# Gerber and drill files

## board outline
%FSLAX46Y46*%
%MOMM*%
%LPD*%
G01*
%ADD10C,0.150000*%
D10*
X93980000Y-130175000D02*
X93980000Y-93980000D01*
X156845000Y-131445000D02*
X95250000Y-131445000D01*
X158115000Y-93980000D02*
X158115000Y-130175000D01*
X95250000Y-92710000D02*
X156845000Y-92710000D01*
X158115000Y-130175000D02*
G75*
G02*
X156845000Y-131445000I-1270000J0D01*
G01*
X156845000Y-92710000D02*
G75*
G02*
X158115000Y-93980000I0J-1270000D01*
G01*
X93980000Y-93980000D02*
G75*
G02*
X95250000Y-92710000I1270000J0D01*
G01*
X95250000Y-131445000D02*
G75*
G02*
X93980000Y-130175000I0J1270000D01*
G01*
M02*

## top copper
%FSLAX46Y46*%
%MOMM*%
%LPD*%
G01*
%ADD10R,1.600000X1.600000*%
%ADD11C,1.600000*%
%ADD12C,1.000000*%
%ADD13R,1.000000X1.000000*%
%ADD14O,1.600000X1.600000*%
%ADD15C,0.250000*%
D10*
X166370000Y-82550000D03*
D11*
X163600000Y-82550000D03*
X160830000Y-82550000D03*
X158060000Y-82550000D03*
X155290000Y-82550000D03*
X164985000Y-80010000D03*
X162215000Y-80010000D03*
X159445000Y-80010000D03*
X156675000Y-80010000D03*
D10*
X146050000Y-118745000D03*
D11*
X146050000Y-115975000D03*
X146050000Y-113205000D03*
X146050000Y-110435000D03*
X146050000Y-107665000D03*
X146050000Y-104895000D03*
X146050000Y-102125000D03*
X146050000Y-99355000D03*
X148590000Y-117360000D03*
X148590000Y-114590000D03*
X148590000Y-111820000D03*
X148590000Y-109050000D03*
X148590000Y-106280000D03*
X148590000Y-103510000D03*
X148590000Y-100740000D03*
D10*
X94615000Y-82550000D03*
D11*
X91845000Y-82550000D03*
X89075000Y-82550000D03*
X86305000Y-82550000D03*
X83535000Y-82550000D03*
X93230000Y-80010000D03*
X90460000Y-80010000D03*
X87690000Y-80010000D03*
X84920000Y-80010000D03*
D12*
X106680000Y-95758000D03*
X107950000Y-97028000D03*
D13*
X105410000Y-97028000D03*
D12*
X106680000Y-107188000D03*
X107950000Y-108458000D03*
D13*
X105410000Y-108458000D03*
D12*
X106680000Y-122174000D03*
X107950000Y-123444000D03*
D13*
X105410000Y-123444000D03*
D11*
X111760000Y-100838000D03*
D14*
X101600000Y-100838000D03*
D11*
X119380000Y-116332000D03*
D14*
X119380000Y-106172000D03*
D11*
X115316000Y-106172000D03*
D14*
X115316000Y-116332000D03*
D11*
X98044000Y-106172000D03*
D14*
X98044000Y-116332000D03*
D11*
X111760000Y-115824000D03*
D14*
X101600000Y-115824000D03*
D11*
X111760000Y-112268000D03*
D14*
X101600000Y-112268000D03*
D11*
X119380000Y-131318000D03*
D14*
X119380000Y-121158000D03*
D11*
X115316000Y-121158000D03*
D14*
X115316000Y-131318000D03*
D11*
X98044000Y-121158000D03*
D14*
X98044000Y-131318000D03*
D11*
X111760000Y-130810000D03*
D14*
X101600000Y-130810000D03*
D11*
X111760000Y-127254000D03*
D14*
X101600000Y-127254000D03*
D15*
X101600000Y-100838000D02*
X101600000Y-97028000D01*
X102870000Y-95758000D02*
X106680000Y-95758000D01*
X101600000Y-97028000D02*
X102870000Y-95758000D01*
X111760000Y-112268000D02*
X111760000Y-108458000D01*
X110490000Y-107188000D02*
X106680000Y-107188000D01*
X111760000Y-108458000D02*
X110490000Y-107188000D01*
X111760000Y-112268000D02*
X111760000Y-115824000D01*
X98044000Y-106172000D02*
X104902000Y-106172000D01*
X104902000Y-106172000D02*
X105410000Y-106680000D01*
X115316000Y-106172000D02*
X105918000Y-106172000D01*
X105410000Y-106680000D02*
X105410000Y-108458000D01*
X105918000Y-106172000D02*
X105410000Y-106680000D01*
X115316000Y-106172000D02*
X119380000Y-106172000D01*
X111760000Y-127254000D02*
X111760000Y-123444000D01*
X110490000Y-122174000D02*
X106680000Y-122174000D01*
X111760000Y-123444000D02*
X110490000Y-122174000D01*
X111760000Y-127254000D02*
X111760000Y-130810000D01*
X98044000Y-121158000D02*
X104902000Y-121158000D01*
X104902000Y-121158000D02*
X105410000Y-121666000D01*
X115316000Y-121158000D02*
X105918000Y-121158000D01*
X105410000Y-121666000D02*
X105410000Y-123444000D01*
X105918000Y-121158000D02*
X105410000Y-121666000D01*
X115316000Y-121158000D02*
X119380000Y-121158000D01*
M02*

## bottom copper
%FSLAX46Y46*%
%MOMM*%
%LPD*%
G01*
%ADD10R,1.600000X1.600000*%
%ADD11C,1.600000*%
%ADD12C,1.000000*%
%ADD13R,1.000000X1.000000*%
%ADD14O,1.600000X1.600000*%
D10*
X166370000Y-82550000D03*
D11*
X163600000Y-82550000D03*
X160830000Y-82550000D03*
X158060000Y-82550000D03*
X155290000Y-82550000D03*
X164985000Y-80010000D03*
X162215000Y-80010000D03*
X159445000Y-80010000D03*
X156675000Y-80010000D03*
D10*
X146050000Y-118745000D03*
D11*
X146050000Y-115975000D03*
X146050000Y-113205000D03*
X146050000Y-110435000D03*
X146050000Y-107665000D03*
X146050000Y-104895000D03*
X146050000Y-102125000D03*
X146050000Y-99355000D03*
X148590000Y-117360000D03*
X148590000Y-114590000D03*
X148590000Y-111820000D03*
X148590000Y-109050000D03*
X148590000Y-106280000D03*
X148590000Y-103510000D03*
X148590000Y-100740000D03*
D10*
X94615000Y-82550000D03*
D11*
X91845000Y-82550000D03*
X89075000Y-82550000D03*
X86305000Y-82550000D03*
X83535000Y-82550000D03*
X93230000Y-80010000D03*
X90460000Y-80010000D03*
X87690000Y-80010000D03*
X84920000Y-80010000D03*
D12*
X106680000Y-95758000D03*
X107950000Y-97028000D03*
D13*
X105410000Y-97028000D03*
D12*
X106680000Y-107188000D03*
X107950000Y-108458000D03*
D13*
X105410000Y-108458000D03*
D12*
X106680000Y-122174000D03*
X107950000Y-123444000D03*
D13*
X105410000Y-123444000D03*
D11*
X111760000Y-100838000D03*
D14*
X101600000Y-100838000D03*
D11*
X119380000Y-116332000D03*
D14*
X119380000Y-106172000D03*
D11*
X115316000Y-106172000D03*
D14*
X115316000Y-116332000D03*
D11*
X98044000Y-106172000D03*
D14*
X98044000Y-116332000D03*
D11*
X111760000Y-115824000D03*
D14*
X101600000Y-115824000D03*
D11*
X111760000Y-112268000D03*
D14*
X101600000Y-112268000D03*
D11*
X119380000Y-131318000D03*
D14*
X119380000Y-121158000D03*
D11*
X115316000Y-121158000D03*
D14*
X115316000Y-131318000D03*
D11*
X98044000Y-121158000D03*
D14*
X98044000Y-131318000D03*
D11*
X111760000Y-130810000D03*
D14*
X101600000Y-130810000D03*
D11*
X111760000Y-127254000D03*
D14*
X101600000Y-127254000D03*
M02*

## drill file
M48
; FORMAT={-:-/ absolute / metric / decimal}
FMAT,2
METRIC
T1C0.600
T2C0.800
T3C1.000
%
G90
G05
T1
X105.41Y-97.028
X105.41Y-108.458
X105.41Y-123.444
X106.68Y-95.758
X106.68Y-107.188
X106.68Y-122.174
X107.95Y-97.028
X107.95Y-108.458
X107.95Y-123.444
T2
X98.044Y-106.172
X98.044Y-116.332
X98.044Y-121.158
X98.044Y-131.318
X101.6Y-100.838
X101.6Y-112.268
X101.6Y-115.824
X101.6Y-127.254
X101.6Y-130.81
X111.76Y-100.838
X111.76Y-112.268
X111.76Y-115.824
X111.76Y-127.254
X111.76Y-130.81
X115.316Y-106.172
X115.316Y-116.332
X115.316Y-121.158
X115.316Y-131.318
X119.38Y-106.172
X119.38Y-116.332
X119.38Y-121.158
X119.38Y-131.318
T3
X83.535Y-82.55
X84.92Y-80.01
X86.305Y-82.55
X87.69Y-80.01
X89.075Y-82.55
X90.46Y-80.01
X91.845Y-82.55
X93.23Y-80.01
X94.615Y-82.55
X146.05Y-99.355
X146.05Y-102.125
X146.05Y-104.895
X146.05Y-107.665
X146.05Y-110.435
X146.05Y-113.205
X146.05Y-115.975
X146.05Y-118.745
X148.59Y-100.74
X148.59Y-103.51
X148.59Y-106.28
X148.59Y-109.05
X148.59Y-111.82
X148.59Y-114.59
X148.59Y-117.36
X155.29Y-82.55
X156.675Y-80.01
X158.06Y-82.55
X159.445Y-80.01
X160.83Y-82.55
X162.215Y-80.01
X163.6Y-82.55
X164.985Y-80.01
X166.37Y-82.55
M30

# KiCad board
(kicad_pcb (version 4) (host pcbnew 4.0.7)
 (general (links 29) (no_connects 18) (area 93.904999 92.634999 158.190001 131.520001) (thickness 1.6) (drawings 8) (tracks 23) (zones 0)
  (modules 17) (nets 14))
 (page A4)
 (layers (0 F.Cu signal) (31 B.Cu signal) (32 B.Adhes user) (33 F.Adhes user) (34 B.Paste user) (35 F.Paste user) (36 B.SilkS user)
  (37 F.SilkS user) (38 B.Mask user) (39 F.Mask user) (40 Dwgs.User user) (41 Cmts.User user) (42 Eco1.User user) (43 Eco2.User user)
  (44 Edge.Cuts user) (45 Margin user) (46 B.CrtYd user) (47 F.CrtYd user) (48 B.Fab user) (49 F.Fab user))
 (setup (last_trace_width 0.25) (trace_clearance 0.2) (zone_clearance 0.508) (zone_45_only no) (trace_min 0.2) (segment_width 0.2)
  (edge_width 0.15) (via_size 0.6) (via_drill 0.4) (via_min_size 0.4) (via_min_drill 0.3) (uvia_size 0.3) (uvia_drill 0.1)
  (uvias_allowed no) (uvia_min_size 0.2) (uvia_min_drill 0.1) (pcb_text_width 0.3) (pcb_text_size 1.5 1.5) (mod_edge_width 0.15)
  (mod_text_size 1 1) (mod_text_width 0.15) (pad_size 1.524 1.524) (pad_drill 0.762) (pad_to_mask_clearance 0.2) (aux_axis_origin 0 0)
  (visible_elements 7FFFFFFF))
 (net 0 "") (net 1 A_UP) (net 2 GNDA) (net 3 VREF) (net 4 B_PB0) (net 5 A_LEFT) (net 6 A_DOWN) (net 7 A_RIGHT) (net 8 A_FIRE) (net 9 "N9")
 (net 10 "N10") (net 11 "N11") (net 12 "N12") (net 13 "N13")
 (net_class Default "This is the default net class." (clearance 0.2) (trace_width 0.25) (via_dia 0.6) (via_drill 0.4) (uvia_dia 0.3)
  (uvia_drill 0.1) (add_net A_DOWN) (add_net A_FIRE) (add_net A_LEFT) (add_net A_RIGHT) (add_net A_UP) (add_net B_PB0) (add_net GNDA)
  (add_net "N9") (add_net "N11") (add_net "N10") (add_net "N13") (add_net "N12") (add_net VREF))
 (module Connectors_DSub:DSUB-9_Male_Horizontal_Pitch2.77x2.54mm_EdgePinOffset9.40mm (layer F.Cu) (at 166.37 82.55 180)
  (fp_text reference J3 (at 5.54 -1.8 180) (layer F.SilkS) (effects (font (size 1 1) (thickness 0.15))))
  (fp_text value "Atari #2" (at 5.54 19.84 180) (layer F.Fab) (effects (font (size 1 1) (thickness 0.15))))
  (pad 1 thru_hole rect (at 0 0 180) (size 1.6 1.6) (drill 1) (layers *.Cu *.Mask))
  (pad 2 thru_hole circle (at 2.77 0 180) (size 1.6 1.6) (drill 1) (layers *.Cu *.Mask))
  (pad 3 thru_hole circle (at 5.54 0 180) (size 1.6 1.6) (drill 1) (layers *.Cu *.Mask))
  (pad 4 thru_hole circle (at 8.31 0 180) (size 1.6 1.6) (drill 1) (layers *.Cu *.Mask))
  (pad 5 thru_hole circle (at 11.08 0 180) (size 1.6 1.6) (drill 1) (layers *.Cu *.Mask))
  (pad 6 thru_hole circle (at 1.385 2.54 180) (size 1.6 1.6) (drill 1) (layers *.Cu *.Mask))
  (pad 7 thru_hole circle (at 4.155 2.54 180) (size 1.6 1.6) (drill 1) (layers *.Cu *.Mask))
  (pad 8 thru_hole circle (at 6.925 2.54 180) (size 1.6 1.6) (drill 1) (layers *.Cu *.Mask))
  (pad 9 thru_hole circle (at 9.695 2.54 180) (size 1.6 1.6) (drill 1) (layers *.Cu *.Mask)))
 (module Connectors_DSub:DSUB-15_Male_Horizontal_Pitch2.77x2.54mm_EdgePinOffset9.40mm (layer F.Cu) (at 146.05 118.745 90)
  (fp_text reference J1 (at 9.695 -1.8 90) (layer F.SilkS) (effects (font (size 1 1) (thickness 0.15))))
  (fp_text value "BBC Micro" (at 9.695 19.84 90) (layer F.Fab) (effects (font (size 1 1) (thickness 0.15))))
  (pad 1 thru_hole rect (at 0 0 90) (size 1.6 1.6) (drill 1) (layers *.Cu *.Mask))
  (pad 2 thru_hole circle (at 2.77 0 90) (size 1.6 1.6) (drill 1) (layers *.Cu *.Mask))
  (pad 3 thru_hole circle (at 5.54 0 90) (size 1.6 1.6) (drill 1) (layers *.Cu *.Mask))
  (pad 4 thru_hole circle (at 8.31 0 90) (size 1.6 1.6) (drill 1) (layers *.Cu *.Mask))
  (pad 5 thru_hole circle (at 11.08 0 90) (size 1.6 1.6) (drill 1) (layers *.Cu *.Mask))
  (pad 6 thru_hole circle (at 13.85 0 90) (size 1.6 1.6) (drill 1) (layers *.Cu *.Mask))
  (pad 7 thru_hole circle (at 16.62 0 90) (size 1.6 1.6) (drill 1) (layers *.Cu *.Mask) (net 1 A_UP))
  (pad 8 thru_hole circle (at 19.39 0 90) (size 1.6 1.6) (drill 1) (layers *.Cu *.Mask) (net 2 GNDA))
  (pad 9 thru_hole circle (at 1.385 2.54 90) (size 1.6 1.6) (drill 1) (layers *.Cu *.Mask))
  (pad 10 thru_hole circle (at 4.155 2.54 90) (size 1.6 1.6) (drill 1) (layers *.Cu *.Mask))
  (pad 11 thru_hole circle (at 6.925 2.54 90) (size 1.6 1.6) (drill 1) (layers *.Cu *.Mask) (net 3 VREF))
  (pad 12 thru_hole circle (at 9.695 2.54 90) (size 1.6 1.6) (drill 1) (layers *.Cu *.Mask))
  (pad 13 thru_hole circle (at 12.465 2.54 90) (size 1.6 1.6) (drill 1) (layers *.Cu *.Mask) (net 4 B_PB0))
  (pad 14 thru_hole circle (at 15.235 2.54 90) (size 1.6 1.6) (drill 1) (layers *.Cu *.Mask))
  (pad 15 thru_hole circle (at 18.005 2.54 90) (size 1.6 1.6) (drill 1) (layers *.Cu *.Mask) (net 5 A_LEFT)))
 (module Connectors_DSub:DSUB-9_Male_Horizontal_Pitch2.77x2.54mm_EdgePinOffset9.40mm (layer F.Cu) (at 94.615 82.55 180)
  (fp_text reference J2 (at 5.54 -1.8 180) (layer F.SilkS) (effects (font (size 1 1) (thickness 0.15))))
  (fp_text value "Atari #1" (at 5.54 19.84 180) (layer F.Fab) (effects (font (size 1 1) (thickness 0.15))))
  (pad 1 thru_hole rect (at 0 0 180) (size 1.6 1.6) (drill 1) (layers *.Cu *.Mask) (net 1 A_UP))
  (pad 2 thru_hole circle (at 2.77 0 180) (size 1.6 1.6) (drill 1) (layers *.Cu *.Mask) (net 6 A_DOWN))
  (pad 3 thru_hole circle (at 5.54 0 180) (size 1.6 1.6) (drill 1) (layers *.Cu *.Mask) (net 5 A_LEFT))
  (pad 4 thru_hole circle (at 8.31 0 180) (size 1.6 1.6) (drill 1) (layers *.Cu *.Mask) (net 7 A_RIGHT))
  (pad 5 thru_hole circle (at 11.08 0 180) (size 1.6 1.6) (drill 1) (layers *.Cu *.Mask))
  (pad 6 thru_hole circle (at 1.385 2.54 180) (size 1.6 1.6) (drill 1) (layers *.Cu *.Mask) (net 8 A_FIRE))
  (pad 7 thru_hole circle (at 4.155 2.54 180) (size 1.6 1.6) (drill 1) (layers *.Cu *.Mask))
  (pad 8 thru_hole circle (at 6.925 2.54 180) (size 1.6 1.6) (drill 1) (layers *.Cu *.Mask) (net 3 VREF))
  (pad 9 thru_hole circle (at 9.695 2.54 180) (size 1.6 1.6) (drill 1) (layers *.Cu *.Mask)))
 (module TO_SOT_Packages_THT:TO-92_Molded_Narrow (layer F.Cu) (at 105.41 97.028)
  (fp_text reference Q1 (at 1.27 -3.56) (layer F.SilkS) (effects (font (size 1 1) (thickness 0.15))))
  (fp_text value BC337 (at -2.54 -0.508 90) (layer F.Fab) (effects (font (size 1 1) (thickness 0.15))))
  (pad 2 thru_hole circle (at 1.27 -1.27 90) (size 1 1) (drill 0.6) (layers *.Cu *.Mask) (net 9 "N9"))
  (pad 3 thru_hole circle (at 2.54 0 90) (size 1 1) (drill 0.6) (layers *.Cu *.Mask) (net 2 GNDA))
  (pad 1 thru_hole rect (at 0 0 90) (size 1 1) (drill 0.6) (layers *.Cu *.Mask) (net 4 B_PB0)))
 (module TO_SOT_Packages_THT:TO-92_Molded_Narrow (layer F.Cu) (at 105.41 108.458)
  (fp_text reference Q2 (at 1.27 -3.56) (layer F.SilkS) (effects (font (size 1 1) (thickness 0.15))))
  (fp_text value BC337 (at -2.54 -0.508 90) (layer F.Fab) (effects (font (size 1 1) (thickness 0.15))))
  (pad 2 thru_hole circle (at 1.27 -1.27 90) (size 1 1) (drill 0.6) (layers *.Cu *.Mask) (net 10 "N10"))
  (pad 3 thru_hole circle (at 2.54 0 90) (size 1 1) (drill 0.6) (layers *.Cu *.Mask) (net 2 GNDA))
  (pad 1 thru_hole rect (at 0 0 90) (size 1 1) (drill 0.6) (layers *.Cu *.Mask) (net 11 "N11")))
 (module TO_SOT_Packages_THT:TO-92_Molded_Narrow (layer F.Cu) (at 105.41 123.444)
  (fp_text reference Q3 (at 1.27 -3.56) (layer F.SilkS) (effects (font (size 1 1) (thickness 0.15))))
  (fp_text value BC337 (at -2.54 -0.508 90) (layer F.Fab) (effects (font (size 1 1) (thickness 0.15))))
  (pad 2 thru_hole circle (at 1.27 -1.27 90) (size 1 1) (drill 0.6) (layers *.Cu *.Mask) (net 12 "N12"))
  (pad 3 thru_hole circle (at 2.54 0 90) (size 1 1) (drill 0.6) (layers *.Cu *.Mask) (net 2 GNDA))
  (pad 1 thru_hole rect (at 0 0 90) (size 1 1) (drill 0.6) (layers *.Cu *.Mask) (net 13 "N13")))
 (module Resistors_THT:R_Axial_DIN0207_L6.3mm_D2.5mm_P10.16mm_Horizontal (layer F.Cu) (at 111.76 100.838 180)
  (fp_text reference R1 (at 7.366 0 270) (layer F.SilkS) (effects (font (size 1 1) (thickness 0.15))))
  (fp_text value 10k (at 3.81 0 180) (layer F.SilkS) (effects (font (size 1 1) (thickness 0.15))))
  (pad 1 thru_hole circle (at 0 0 180) (size 1.6 1.6) (drill 0.8) (layers *.Cu *.Mask) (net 8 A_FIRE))
  (pad 2 thru_hole oval (at 10.16 0 180) (size 1.6 1.6) (drill 0.8) (layers *.Cu *.Mask) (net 9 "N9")))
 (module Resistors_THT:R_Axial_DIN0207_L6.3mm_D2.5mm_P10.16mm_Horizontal (layer F.Cu) (at 119.38 116.332 90)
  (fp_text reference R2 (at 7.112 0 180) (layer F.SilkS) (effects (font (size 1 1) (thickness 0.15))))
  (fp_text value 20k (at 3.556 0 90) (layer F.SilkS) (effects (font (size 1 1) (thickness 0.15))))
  (pad 1 thru_hole circle (at 0 0 90) (size 1.6 1.6) (drill 0.8) (layers *.Cu *.Mask) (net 3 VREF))
  (pad 2 thru_hole oval (at 10.16 0 90) (size 1.6 1.6) (drill 0.8) (layers *.Cu *.Mask) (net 11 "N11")))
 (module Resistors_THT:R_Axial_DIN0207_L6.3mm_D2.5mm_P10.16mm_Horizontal (layer F.Cu) (at 115.316 106.172 270)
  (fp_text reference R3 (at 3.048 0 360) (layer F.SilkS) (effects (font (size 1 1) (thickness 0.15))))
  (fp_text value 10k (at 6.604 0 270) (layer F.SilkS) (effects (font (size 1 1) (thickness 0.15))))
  (pad 1 thru_hole circle (at 0 0 270) (size 1.6 1.6) (drill 0.8) (layers *.Cu *.Mask) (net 11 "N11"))
  (pad 2 thru_hole oval (at 10.16 0 270) (size 1.6 1.6) (drill 0.8) (layers *.Cu *.Mask) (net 5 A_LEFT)))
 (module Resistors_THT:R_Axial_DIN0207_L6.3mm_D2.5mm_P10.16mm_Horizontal (layer F.Cu) (at 98.044 106.172 270)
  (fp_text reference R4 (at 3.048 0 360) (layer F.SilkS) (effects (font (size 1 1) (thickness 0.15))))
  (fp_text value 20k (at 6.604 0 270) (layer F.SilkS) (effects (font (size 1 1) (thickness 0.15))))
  (pad 1 thru_hole circle (at 0 0 270) (size 1.6 1.6) (drill 0.8) (layers *.Cu *.Mask) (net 11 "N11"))
  (pad 2 thru_hole oval (at 10.16 0 270) (size 1.6 1.6) (drill 0.8) (layers *.Cu *.Mask) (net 2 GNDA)))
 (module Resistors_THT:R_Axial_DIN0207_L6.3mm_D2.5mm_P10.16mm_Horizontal (layer F.Cu) (at 111.76 115.824 180)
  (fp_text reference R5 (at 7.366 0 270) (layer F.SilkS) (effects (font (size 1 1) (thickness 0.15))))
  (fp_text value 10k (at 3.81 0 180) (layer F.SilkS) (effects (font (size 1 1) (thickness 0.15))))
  (pad 1 thru_hole circle (at 0 0 180) (size 1.6 1.6) (drill 0.8) (layers *.Cu *.Mask) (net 10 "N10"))
  (pad 2 thru_hole oval (at 10.16 0 180) (size 1.6 1.6) (drill 0.8) (layers *.Cu *.Mask) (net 7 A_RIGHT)))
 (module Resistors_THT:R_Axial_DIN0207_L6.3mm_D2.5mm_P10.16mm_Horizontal (layer F.Cu) (at 111.76 112.268 180)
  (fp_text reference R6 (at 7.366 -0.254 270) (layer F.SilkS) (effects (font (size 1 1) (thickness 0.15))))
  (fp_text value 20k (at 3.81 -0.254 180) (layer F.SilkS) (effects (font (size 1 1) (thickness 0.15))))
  (pad 1 thru_hole circle (at 0 0 180) (size 1.6 1.6) (drill 0.8) (layers *.Cu *.Mask) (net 10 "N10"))
  (pad 2 thru_hole oval (at 10.16 0 180) (size 1.6 1.6) (drill 0.8) (layers *.Cu *.Mask) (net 2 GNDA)))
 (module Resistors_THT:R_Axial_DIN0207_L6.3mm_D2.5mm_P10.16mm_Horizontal (layer F.Cu) (at 119.38 131.318 90)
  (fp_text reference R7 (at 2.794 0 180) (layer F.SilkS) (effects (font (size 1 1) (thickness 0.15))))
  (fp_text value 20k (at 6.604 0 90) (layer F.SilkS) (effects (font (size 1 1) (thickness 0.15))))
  (pad 1 thru_hole circle (at 0 0 90) (size 1.6 1.6) (drill 0.8) (layers *.Cu *.Mask) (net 3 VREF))
  (pad 2 thru_hole oval (at 10.16 0 90) (size 1.6 1.6) (drill 0.8) (layers *.Cu *.Mask) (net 13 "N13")))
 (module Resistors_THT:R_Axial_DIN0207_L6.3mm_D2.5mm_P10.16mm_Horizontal (layer F.Cu) (at 115.316 121.158 270)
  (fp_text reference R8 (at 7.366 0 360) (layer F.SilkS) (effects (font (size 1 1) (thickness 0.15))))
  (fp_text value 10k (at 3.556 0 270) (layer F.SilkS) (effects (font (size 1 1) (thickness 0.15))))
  (pad 1 thru_hole circle (at 0 0 270) (size 1.6 1.6) (drill 0.8) (layers *.Cu *.Mask) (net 13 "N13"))
  (pad 2 thru_hole oval (at 10.16 0 270) (size 1.6 1.6) (drill 0.8) (layers *.Cu *.Mask) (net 1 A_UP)))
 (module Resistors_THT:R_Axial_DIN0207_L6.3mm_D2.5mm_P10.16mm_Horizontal (layer F.Cu) (at 98.044 121.158 270)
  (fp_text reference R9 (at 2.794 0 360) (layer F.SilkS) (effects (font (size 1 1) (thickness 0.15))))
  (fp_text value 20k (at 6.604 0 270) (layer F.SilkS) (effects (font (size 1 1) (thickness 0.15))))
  (pad 1 thru_hole circle (at 0 0 270) (size 1.6 1.6) (drill 0.8) (layers *.Cu *.Mask) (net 13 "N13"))
  (pad 2 thru_hole oval (at 10.16 0 270) (size 1.6 1.6) (drill 0.8) (layers *.Cu *.Mask) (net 2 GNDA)))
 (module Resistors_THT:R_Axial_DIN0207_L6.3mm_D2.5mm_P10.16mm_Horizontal (layer F.Cu) (at 111.76 130.81 180)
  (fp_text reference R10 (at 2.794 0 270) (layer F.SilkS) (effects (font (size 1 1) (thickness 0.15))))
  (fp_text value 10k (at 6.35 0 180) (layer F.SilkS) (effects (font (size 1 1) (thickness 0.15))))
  (pad 1 thru_hole circle (at 0 0 180) (size 1.6 1.6) (drill 0.8) (layers *.Cu *.Mask) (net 12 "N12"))
  (pad 2 thru_hole oval (at 10.16 0 180) (size 1.6 1.6) (drill 0.8) (layers *.Cu *.Mask) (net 6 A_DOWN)))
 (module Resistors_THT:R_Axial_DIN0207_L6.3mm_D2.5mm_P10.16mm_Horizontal (layer F.Cu) (at 111.76 127.254 180)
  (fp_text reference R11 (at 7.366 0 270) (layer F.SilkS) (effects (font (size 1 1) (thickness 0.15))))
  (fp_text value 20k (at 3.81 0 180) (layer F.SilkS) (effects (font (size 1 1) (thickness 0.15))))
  (pad 1 thru_hole circle (at 0 0 180) (size 1.6 1.6) (drill 0.8) (layers *.Cu *.Mask) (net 12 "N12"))
  (pad 2 thru_hole oval (at 10.16 0 180) (size 1.6 1.6) (drill 0.8) (layers *.Cu *.Mask) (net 2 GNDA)))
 (gr_line (start 93.98 130.175) (end 93.98 93.98) (angle 90) (layer Edge.Cuts) (width 0.15))
 (gr_line (start 156.845 131.445) (end 95.25 131.445) (angle 90) (layer Edge.Cuts) (width 0.15))
 (gr_line (start 158.115 93.98) (end 158.115 130.175) (angle 90) (layer Edge.Cuts) (width 0.15))
 (gr_line (start 95.25 92.71) (end 156.845 92.71) (angle 90) (layer Edge.Cuts) (width 0.15))
 (gr_arc (start 156.845 130.175) (end 158.115 130.175) (angle 90) (layer Edge.Cuts) (width 0.15))
 (gr_arc (start 156.845 93.98) (end 156.845 92.71) (angle 90) (layer Edge.Cuts) (width 0.15))
 (gr_arc (start 95.25 93.98) (end 93.98 93.98) (angle 90) (layer Edge.Cuts) (width 0.15))
 (gr_arc (start 95.25 130.175) (end 95.25 131.445) (angle 90) (layer Edge.Cuts) (width 0.15))
 (segment (start 101.6 100.838) (end 101.6 97.028) (width 0.25) (layer F.Cu) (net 9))
 (segment (start 102.87 95.758) (end 106.68 95.758) (width 0.25) (layer F.Cu) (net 9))
 (segment (start 101.6 97.028) (end 102.87 95.758) (width 0.25) (layer F.Cu) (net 9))
 (segment (start 111.76 112.268) (end 111.76 108.458) (width 0.25) (layer F.Cu) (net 10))
 (segment (start 110.49 107.188) (end 106.68 107.188) (width 0.25) (layer F.Cu) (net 10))
 (segment (start 111.76 108.458) (end 110.49 107.188) (width 0.25) (layer F.Cu) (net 10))
 (segment (start 111.76 112.268) (end 111.76 115.824) (width 0.25) (layer F.Cu) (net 10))
 (segment (start 98.044 106.172) (end 104.902 106.172) (width 0.25) (layer F.Cu) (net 11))
 (segment (start 104.902 106.172) (end 105.41 106.68) (width 0.25) (layer F.Cu) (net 11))
 (segment (start 115.316 106.172) (end 105.918 106.172) (width 0.25) (layer F.Cu) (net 11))
 (segment (start 105.41 106.68) (end 105.41 108.458) (width 0.25) (layer F.Cu) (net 11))
 (segment (start 105.918 106.172) (end 105.41 106.68) (width 0.25) (layer F.Cu) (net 11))
 (segment (start 115.316 106.172) (end 119.38 106.172) (width 0.25) (layer F.Cu) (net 11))
 (segment (start 111.76 127.254) (end 111.76 123.444) (width 0.25) (layer F.Cu) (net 12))
 (segment (start 110.49 122.174) (end 106.68 122.174) (width 0.25) (layer F.Cu) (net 12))
 (segment (start 111.76 123.444) (end 110.49 122.174) (width 0.25) (layer F.Cu) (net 12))
 (segment (start 111.76 127.254) (end 111.76 130.81) (width 0.25) (layer F.Cu) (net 12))
 (segment (start 98.044 121.158) (end 104.902 121.158) (width 0.25) (layer F.Cu) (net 13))
 (segment (start 104.902 121.158) (end 105.41 121.666) (width 0.25) (layer F.Cu) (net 13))
 (segment (start 115.316 121.158) (end 105.918 121.158) (width 0.25) (layer F.Cu) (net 13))
 (segment (start 105.41 121.666) (end 105.41 123.444) (width 0.25) (layer F.Cu) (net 13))
 (segment (start 105.918 121.158) (end 105.41 121.666) (width 0.25) (layer F.Cu) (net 13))
 (segment (start 115.316 121.158) (end 119.38 121.158) (width 0.25) (layer F.Cu) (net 13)))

